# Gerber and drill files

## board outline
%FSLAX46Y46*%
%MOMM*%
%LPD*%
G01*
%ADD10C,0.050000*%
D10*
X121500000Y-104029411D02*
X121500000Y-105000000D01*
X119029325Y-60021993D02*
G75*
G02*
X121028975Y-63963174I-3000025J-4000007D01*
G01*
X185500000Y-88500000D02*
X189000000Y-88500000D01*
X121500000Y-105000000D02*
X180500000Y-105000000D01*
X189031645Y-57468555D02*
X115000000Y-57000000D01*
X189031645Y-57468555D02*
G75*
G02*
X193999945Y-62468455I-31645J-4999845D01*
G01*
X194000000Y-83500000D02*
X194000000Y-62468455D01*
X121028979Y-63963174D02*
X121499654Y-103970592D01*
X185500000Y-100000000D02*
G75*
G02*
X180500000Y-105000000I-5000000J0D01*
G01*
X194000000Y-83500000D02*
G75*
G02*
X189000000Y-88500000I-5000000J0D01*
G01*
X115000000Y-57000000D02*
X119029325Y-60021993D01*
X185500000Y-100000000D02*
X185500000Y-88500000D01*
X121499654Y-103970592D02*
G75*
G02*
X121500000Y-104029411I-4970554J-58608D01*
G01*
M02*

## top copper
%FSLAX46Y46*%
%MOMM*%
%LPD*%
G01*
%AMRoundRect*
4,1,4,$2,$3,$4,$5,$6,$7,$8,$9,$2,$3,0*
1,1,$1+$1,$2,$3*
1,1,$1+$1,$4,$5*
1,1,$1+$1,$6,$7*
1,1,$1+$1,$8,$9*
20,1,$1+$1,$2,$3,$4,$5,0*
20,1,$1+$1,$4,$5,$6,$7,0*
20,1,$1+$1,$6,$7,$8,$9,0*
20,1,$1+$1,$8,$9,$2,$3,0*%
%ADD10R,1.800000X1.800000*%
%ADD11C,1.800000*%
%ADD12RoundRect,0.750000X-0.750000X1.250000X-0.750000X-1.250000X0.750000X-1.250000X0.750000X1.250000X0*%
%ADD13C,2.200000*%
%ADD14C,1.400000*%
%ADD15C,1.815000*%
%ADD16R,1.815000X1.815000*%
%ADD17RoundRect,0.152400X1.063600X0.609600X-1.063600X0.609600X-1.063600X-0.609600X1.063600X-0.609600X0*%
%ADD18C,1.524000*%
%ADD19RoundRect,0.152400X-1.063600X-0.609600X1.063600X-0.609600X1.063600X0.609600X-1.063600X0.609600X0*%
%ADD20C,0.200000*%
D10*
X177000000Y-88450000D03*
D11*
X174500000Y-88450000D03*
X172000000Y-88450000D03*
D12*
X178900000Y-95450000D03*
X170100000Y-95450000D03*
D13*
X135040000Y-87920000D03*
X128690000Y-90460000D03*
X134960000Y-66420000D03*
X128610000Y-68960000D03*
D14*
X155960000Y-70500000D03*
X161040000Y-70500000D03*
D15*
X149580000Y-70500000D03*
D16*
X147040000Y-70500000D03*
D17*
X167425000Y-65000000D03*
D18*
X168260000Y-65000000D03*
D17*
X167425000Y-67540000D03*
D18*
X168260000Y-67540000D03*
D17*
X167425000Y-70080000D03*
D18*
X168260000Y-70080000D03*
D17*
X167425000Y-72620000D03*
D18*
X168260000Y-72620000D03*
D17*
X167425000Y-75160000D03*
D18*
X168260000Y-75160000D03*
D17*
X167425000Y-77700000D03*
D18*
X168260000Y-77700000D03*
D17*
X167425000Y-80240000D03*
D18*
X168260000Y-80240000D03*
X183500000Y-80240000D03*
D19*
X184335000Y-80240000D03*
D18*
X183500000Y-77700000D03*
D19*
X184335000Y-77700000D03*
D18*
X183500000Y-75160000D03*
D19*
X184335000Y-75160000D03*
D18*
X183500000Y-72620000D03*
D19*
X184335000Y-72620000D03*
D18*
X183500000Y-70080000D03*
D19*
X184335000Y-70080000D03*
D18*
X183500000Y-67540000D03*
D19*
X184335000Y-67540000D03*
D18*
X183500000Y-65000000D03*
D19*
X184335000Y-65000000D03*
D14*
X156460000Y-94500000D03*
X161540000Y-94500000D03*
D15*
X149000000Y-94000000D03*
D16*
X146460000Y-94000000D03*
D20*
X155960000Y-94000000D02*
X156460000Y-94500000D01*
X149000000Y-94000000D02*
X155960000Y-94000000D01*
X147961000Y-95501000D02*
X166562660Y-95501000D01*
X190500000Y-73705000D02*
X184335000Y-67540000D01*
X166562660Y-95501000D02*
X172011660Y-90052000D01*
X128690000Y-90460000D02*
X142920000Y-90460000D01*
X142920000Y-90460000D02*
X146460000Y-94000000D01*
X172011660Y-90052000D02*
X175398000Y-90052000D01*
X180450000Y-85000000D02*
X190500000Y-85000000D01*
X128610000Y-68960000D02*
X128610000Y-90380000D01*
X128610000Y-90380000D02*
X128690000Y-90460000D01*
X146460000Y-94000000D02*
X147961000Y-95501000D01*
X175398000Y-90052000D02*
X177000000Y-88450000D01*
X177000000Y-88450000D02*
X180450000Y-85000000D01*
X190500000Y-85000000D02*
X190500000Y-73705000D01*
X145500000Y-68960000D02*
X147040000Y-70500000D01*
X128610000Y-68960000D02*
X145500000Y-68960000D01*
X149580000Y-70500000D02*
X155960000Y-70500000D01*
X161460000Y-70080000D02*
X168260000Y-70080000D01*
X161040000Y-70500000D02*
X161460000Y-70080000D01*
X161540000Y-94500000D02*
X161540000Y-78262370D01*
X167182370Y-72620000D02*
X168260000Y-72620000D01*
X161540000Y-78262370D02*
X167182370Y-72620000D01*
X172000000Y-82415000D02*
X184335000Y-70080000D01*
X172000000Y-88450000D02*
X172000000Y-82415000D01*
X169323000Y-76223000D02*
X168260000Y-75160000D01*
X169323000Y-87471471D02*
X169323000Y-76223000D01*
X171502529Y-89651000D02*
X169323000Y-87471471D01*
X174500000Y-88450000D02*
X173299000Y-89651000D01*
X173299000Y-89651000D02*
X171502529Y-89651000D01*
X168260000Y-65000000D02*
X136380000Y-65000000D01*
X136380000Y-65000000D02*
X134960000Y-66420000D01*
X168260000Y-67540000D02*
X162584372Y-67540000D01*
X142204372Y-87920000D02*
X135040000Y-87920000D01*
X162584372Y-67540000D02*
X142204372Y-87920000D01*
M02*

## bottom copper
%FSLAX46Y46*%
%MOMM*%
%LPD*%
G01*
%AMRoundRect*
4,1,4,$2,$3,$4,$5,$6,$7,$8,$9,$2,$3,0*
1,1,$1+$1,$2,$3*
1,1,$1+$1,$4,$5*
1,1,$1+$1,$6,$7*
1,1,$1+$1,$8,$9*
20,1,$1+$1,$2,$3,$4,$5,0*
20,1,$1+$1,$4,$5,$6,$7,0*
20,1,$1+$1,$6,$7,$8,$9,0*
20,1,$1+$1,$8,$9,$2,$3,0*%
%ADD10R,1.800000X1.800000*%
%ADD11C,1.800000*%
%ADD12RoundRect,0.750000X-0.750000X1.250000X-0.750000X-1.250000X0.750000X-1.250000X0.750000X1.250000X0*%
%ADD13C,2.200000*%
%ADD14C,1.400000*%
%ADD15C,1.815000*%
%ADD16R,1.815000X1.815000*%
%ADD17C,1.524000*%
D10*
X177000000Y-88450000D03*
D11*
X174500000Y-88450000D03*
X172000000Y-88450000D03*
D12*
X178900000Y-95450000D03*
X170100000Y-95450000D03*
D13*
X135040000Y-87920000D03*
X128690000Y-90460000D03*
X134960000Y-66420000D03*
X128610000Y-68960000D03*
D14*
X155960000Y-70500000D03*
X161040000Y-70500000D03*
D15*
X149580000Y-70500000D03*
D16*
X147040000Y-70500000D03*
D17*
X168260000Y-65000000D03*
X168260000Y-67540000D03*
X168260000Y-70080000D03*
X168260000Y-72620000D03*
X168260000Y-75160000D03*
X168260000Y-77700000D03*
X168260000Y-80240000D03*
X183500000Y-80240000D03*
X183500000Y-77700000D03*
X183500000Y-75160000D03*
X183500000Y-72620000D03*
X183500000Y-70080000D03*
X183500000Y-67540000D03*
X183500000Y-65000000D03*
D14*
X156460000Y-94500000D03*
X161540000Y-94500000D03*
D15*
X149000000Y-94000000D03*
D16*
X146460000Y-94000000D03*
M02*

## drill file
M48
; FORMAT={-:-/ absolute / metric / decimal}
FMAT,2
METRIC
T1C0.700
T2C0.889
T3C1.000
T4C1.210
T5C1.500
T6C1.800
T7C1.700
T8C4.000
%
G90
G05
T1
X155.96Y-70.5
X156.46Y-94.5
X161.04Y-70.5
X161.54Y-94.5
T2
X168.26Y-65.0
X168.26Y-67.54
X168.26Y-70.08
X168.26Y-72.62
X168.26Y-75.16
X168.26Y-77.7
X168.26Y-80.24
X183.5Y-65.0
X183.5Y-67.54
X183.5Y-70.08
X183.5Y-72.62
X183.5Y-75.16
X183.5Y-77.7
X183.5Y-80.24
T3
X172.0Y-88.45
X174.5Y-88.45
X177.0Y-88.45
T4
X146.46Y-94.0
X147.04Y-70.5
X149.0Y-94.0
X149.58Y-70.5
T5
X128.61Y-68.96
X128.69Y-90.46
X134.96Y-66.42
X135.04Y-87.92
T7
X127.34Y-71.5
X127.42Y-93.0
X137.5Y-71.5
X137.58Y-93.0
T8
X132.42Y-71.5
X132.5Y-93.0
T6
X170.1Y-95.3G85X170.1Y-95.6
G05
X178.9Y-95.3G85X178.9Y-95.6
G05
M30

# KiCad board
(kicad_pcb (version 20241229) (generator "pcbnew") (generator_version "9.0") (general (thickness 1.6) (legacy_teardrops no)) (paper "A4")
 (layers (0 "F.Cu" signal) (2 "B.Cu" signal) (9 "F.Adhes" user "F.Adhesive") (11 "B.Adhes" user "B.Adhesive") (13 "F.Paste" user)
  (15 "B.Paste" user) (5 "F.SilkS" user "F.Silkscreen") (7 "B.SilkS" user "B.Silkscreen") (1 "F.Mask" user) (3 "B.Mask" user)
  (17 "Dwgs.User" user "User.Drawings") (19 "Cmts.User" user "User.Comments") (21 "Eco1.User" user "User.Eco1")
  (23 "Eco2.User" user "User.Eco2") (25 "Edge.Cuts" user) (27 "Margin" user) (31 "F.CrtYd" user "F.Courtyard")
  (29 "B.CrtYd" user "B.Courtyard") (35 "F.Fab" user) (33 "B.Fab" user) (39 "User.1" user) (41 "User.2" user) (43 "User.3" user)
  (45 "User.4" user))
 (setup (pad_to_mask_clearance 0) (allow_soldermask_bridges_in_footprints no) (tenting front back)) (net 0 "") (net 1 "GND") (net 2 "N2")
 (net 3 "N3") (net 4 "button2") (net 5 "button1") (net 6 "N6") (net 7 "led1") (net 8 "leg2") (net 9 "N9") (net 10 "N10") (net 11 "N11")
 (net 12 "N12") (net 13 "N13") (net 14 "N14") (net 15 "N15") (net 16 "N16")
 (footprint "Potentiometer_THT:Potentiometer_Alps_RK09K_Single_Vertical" (layer "F.Cu") (at 177 88.45 -90)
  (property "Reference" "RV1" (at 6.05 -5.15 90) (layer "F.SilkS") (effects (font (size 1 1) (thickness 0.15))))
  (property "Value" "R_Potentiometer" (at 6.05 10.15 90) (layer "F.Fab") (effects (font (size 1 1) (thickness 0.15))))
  (pad "1" thru_hole rect (at 0 0 270) (size 1.8 1.8) (drill 1) (layers "*.Cu" "*.Mask") (remove_unused_layers no) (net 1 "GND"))
  (pad "2" thru_hole circle (at 0 2.5 270) (size 1.8 1.8) (drill 1) (layers "*.Cu" "*.Mask") (remove_unused_layers no) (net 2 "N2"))
  (pad "3" thru_hole circle (at 0 5 270) (size 1.8 1.8) (drill 1) (layers "*.Cu" "*.Mask") (remove_unused_layers no) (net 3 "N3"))
  (pad "MP" thru_hole roundrect (at 7 -1.9 270) (size 4 3) (drill oval 2.1 1.8) (layers "*.Cu" "*.Mask") (remove_unused_layers no)
   (roundrect_rratio 0.25))
  (pad "MP" thru_hole roundrect (at 7 6.9 270) (size 4 3) (drill oval 2.1 1.8) (layers "*.Cu" "*.Mask") (remove_unused_layers no)
   (roundrect_rratio 0.25)))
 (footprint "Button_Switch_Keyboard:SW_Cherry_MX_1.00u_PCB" (layer "F.Cu") (at 135.04 87.92)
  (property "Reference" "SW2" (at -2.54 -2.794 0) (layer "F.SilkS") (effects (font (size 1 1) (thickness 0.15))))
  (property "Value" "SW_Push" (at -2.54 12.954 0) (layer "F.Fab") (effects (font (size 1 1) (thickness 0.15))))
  (pad "" np_thru_hole circle (at -7.62 5.08) (size 1.7 1.7) (drill 1.7) (layers "*.Cu" "*.Mask"))
  (pad "" np_thru_hole circle (at -2.54 5.08) (size 4 4) (drill 4) (layers "*.Cu" "*.Mask"))
  (pad "" np_thru_hole circle (at 2.54 5.08) (size 1.7 1.7) (drill 1.7) (layers "*.Cu" "*.Mask"))
  (pad "1" thru_hole circle (at 0 0) (size 2.2 2.2) (drill 1.5) (layers "*.Cu" "*.Mask") (remove_unused_layers no) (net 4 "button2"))
  (pad "2" thru_hole circle (at -6.35 2.54) (size 2.2 2.2) (drill 1.5) (layers "*.Cu" "*.Mask") (remove_unused_layers no) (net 1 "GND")))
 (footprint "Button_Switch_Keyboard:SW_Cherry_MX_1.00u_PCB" (layer "F.Cu") (at 134.96 66.42)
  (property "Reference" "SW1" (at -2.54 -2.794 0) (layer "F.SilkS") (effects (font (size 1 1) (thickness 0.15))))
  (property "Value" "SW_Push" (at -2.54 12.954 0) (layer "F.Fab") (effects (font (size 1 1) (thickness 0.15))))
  (pad "" np_thru_hole circle (at -7.62 5.08) (size 1.7 1.7) (drill 1.7) (layers "*.Cu" "*.Mask"))
  (pad "" np_thru_hole circle (at -2.54 5.08) (size 4 4) (drill 4) (layers "*.Cu" "*.Mask"))
  (pad "" np_thru_hole circle (at 2.54 5.08) (size 1.7 1.7) (drill 1.7) (layers "*.Cu" "*.Mask"))
  (pad "1" thru_hole circle (at 0 0) (size 2.2 2.2) (drill 1.5) (layers "*.Cu" "*.Mask") (remove_unused_layers no) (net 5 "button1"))
  (pad "2" thru_hole circle (at -6.35 2.54) (size 2.2 2.2) (drill 1.5) (layers "*.Cu" "*.Mask") (remove_unused_layers no) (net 1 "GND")))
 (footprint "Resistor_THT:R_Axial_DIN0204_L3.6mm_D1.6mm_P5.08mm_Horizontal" (layer "F.Cu") (at 155.96 70.5)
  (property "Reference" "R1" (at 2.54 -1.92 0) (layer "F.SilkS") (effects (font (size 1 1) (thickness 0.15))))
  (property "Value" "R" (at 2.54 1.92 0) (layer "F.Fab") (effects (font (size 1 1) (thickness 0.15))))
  (pad "1" thru_hole circle (at 0 0) (size 1.4 1.4) (drill 0.7) (layers "*.Cu" "*.Mask") (remove_unused_layers no) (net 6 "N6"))
  (pad "2" thru_hole circle (at 5.08 0) (size 1.4 1.4) (drill 0.7) (layers "*.Cu" "*.Mask") (remove_unused_layers no) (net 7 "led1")))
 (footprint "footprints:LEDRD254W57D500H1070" (layer "F.Cu") (at 148.31 70.5)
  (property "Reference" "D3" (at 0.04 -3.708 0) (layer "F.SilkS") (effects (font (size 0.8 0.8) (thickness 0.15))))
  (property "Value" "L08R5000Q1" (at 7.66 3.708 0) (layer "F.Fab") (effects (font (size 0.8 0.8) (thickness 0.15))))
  (pad "A" thru_hole circle (at 1.27 0) (size 1.815 1.815) (drill 1.21) (layers "*.Cu" "*.Mask") (remove_unused_layers no) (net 6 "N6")
   (solder_mask_margin 0.102))
  (pad "C" thru_hole rect (at -1.27 0) (size 1.815 1.815) (drill 1.21) (layers "*.Cu" "*.Mask") (remove_unused_layers no) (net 1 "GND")
   (solder_mask_margin 0.102)))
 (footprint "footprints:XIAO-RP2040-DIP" (layer "F.Cu") (at 175.88 72.62 90)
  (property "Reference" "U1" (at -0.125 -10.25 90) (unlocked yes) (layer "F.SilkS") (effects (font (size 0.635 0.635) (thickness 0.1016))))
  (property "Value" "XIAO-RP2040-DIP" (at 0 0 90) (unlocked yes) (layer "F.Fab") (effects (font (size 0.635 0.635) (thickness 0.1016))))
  (pad "1" smd roundrect (at 7.62 -8.455 180) (size 2.432 1.524) (layers "F.Cu" "F.Mask") (roundrect_rratio 0.1) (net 5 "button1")
   (thermal_bridge_angle 45))
  (pad "1" thru_hole circle (at 7.62 -7.62 180) (size 1.524 1.524) (drill 0.889) (layers "*.Cu" "*.Mask") (remove_unused_layers no)
   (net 5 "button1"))
  (pad "2" smd roundrect (at 5.08 -8.455 180) (size 2.432 1.524) (layers "F.Cu" "F.Mask") (roundrect_rratio 0.1) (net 4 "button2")
   (thermal_bridge_angle 45))
  (pad "2" thru_hole circle (at 5.08 -7.62 180) (size 1.524 1.524) (drill 0.889) (layers "*.Cu" "*.Mask") (remove_unused_layers no)
   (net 4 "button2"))
  (pad "3" smd roundrect (at 2.54 -8.455 180) (size 2.432 1.524) (layers "F.Cu" "F.Mask") (roundrect_rratio 0.1) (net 7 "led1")
   (thermal_bridge_angle 45))
  (pad "3" thru_hole circle (at 2.54 -7.62 180) (size 1.524 1.524) (drill 0.889) (layers "*.Cu" "*.Mask") (remove_unused_layers no)
   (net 7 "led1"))
  (pad "4" smd roundrect (at 0 -8.455 180) (size 2.432 1.524) (layers "F.Cu" "F.Mask") (roundrect_rratio 0.1) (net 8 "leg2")
   (thermal_bridge_angle 45))
  (pad "4" thru_hole circle (at 0 -7.62 180) (size 1.524 1.524) (drill 0.889) (layers "*.Cu" "*.Mask") (remove_unused_layers no)
   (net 8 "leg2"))
  (pad "5" smd roundrect (at -2.54 -8.455 180) (size 2.432 1.524) (layers "F.Cu" "F.Mask") (roundrect_rratio 0.1) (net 2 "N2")
   (thermal_bridge_angle 45))
  (pad "5" thru_hole circle (at -2.54 -7.62 180) (size 1.524 1.524) (drill 0.889) (layers "*.Cu" "*.Mask") (remove_unused_layers no)
   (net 2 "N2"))
  (pad "6" smd roundrect (at -5.08 -8.455 180) (size 2.432 1.524) (layers "F.Cu" "F.Mask") (roundrect_rratio 0.1) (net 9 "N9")
   (thermal_bridge_angle 45))
  (pad "6" thru_hole circle (at -5.08 -7.62 180) (size 1.524 1.524) (drill 0.889) (layers "*.Cu" "*.Mask") (remove_unused_layers no)
   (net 9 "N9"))
  (pad "7" smd roundrect (at -7.62 -8.455 180) (size 2.432 1.524) (layers "F.Cu" "F.Mask") (roundrect_rratio 0.1) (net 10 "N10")
   (thermal_bridge_angle 45))
  (pad "7" thru_hole circle (at -7.62 -7.62 180) (size 1.524 1.524) (drill 0.889) (layers "*.Cu" "*.Mask") (remove_unused_layers no)
   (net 10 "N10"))
  (pad "8" thru_hole circle (at -7.62 7.62) (size 1.524 1.524) (drill 0.889) (layers "*.Cu" "*.Mask") (remove_unused_layers no)
   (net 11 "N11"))
  (pad "8" smd roundrect (at -7.62 8.455) (size 2.432 1.524) (layers "F.Cu" "F.Mask") (roundrect_rratio 0.1) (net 11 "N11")
   (thermal_bridge_angle 45))
  (pad "9" thru_hole circle (at -5.08 7.62) (size 1.524 1.524) (drill 0.889) (layers "*.Cu" "*.Mask") (remove_unused_layers no)
   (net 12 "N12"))
  (pad "9" smd roundrect (at -5.08 8.455) (size 2.432 1.524) (layers "F.Cu" "F.Mask") (roundrect_rratio 0.1) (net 12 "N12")
   (thermal_bridge_angle 45))
  (pad "10" thru_hole circle (at -2.54 7.62) (size 1.524 1.524) (drill 0.889) (layers "*.Cu" "*.Mask") (remove_unused_layers no)
   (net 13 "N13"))
  (pad "10" smd roundrect (at -2.54 8.455) (size 2.432 1.524) (layers "F.Cu" "F.Mask") (roundrect_rratio 0.1) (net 13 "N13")
   (thermal_bridge_angle 45))
  (pad "11" thru_hole circle (at 0 7.62) (size 1.524 1.524) (drill 0.889) (layers "*.Cu" "*.Mask") (remove_unused_layers no) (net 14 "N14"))
  (pad "11" smd roundrect (at 0 8.455) (size 2.432 1.524) (layers "F.Cu" "F.Mask") (roundrect_rratio 0.1) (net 14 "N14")
   (thermal_bridge_angle 45))
  (pad "12" thru_hole circle (at 2.54 7.62) (size 1.524 1.524) (drill 0.889) (layers "*.Cu" "*.Mask") (remove_unused_layers no) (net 3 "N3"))
  (pad "12" smd roundrect (at 2.54 8.455) (size 2.432 1.524) (layers "F.Cu" "F.Mask") (roundrect_rratio 0.1) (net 3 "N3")
   (thermal_bridge_angle 45))
  (pad "13" thru_hole circle (at 5.08 7.62) (size 1.524 1.524) (drill 0.889) (layers "*.Cu" "*.Mask") (remove_unused_layers no)
   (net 1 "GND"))
  (pad "13" smd roundrect (at 5.08 8.455) (size 2.432 1.524) (layers "F.Cu" "F.Mask") (roundrect_rratio 0.1) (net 1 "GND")
   (thermal_bridge_angle 45))
  (pad "14" thru_hole circle (at 7.62 7.62) (size 1.524 1.524) (drill 0.889) (layers "*.Cu" "*.Mask") (remove_unused_layers no)
   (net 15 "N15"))
  (pad "14" smd roundrect (at 7.62 8.455) (size 2.432 1.524) (layers "F.Cu" "F.Mask") (roundrect_rratio 0.1) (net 15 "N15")
   (thermal_bridge_angle 45)))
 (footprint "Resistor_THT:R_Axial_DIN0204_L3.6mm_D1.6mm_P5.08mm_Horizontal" (layer "F.Cu") (at 156.46 94.5)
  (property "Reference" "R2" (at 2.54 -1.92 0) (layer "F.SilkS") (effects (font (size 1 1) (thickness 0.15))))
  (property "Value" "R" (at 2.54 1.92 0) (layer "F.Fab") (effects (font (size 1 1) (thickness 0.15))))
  (pad "1" thru_hole circle (at 0 0) (size 1.4 1.4) (drill 0.7) (layers "*.Cu" "*.Mask") (remove_unused_layers no) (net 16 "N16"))
  (pad "2" thru_hole circle (at 5.08 0) (size 1.4 1.4) (drill 0.7) (layers "*.Cu" "*.Mask") (remove_unused_layers no) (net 8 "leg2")))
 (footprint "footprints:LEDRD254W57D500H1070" (layer "F.Cu") (at 147.73 94)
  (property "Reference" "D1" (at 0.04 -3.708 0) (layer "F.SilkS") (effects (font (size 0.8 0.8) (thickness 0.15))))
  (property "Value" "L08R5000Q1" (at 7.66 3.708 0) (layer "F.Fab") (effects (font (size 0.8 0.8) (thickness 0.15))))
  (pad "A" thru_hole circle (at 1.27 0) (size 1.815 1.815) (drill 1.21) (layers "*.Cu" "*.Mask") (remove_unused_layers no) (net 16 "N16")
   (solder_mask_margin 0.102))
  (pad "C" thru_hole rect (at -1.27 0) (size 1.815 1.815) (drill 1.21) (layers "*.Cu" "*.Mask") (remove_unused_layers no) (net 1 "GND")
   (solder_mask_margin 0.102)))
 (gr_line (start 121.5 104.029411) (end 121.5 105) (stroke (width 0.05) (type default)) (layer "Edge.Cuts"))
 (gr_arc (start 119.029325 60.021993) (mid 120.488231 61.759659) (end 121.028979 63.963174) (stroke (width 0.05) (type default))
  (layer "Edge.Cuts"))
 (gr_line (start 185.5 88.5) (end 189 88.5) (stroke (width 0.05) (type default)) (layer "Edge.Cuts"))
 (gr_line (start 121.5 105) (end 180.5 105) (stroke (width 0.05) (type default)) (layer "Edge.Cuts"))
 (gr_line (start 189.031645 57.468555) (end 115 57) (stroke (width 0.05) (type default)) (layer "Edge.Cuts"))
 (gr_arc (start 189.031645 57.468555) (mid 192.546721 58.944124) (end 194 62.468455) (stroke (width 0.05) (type default))
  (layer "Edge.Cuts"))
 (gr_line (start 194 83.5) (end 194 62.468455) (stroke (width 0.05) (type default)) (layer "Edge.Cuts"))
 (gr_line (start 121.028979 63.963174) (end 121.499654 103.970592) (stroke (width 0.05) (type default)) (layer "Edge.Cuts"))
 (gr_arc (start 185.5 100) (mid 184.035534 103.535534) (end 180.5 105) (stroke (width 0.05) (type default)) (layer "Edge.Cuts"))
 (gr_arc (start 194 83.5) (mid 192.535534 87.035534) (end 189 88.5) (stroke (width 0.05) (type default)) (layer "Edge.Cuts"))
 (gr_line (start 115 57) (end 119.029325 60.021993) (stroke (width 0.05) (type default)) (layer "Edge.Cuts"))
 (gr_line (start 185.5 100) (end 185.5 88.5) (stroke (width 0.05) (type default)) (layer "Edge.Cuts"))
 (gr_arc (start 121.499654 103.970592) (mid 121.499914 104.000001) (end 121.5 104.029411) (stroke (width 0.05) (type default))
  (layer "Edge.Cuts"))
 (segment (start 155.96 94) (end 156.46 94.5) (width 0.2) (layer "F.Cu") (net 16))
 (segment (start 149 94) (end 155.96 94) (width 0.2) (layer "F.Cu") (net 16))
 (segment (start 147.961 95.501) (end 166.56266 95.501) (width 0.2) (layer "F.Cu") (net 1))
 (segment (start 190.5 73.705) (end 184.335 67.54) (width 0.2) (layer "F.Cu") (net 1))
 (segment (start 166.56266 95.501) (end 172.01166 90.052) (width 0.2) (layer "F.Cu") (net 1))
 (segment (start 128.69 90.46) (end 142.92 90.46) (width 0.2) (layer "F.Cu") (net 1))
 (segment (start 142.92 90.46) (end 146.46 94) (width 0.2) (layer "F.Cu") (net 1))
 (segment (start 172.01166 90.052) (end 175.398 90.052) (width 0.2) (layer "F.Cu") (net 1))
 (segment (start 180.45 85) (end 190.5 85) (width 0.2) (layer "F.Cu") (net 1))
 (segment (start 128.61 68.96) (end 128.61 90.38) (width 0.2) (layer "F.Cu") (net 1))
 (segment (start 128.61 90.38) (end 128.69 90.46) (width 0.2) (layer "F.Cu") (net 1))
 (segment (start 146.46 94) (end 147.961 95.501) (width 0.2) (layer "F.Cu") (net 1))
 (segment (start 175.398 90.052) (end 177 88.45) (width 0.2) (layer "F.Cu") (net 1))
 (segment (start 177 88.45) (end 180.45 85) (width 0.2) (layer "F.Cu") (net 1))
 (segment (start 190.5 85) (end 190.5 73.705) (width 0.2) (layer "F.Cu") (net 1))
 (segment (start 145.5 68.96) (end 147.04 70.5) (width 0.2) (layer "F.Cu") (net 1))
 (segment (start 128.61 68.96) (end 145.5 68.96) (width 0.2) (layer "F.Cu") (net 1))
 (segment (start 149.58 70.5) (end 155.96 70.5) (width 0.2) (layer "F.Cu") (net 6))
 (segment (start 161.46 70.08) (end 168.26 70.08) (width 0.2) (layer "F.Cu") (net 7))
 (segment (start 161.04 70.5) (end 161.46 70.08) (width 0.2) (layer "F.Cu") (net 7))
 (segment (start 161.54 94.5) (end 161.54 78.26237) (width 0.2) (layer "F.Cu") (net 8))
 (segment (start 167.18237 72.62) (end 168.26 72.62) (width 0.2) (layer "F.Cu") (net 8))
 (segment (start 161.54 78.26237) (end 167.18237 72.62) (width 0.2) (layer "F.Cu") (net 8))
 (segment (start 172 82.415) (end 184.335 70.08) (width 0.2) (layer "F.Cu") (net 3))
 (segment (start 172 88.45) (end 172 82.415) (width 0.2) (layer "F.Cu") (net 3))
 (segment (start 169.323 76.223) (end 168.26 75.16) (width 0.2) (layer "F.Cu") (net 2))
 (segment (start 169.323 87.471471) (end 169.323 76.223) (width 0.2) (layer "F.Cu") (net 2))
 (segment (start 171.502529 89.651) (end 169.323 87.471471) (width 0.2) (layer "F.Cu") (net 2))
 (segment (start 174.5 88.45) (end 173.299 89.651) (width 0.2) (layer "F.Cu") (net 2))
 (segment (start 173.299 89.651) (end 171.502529 89.651) (width 0.2) (layer "F.Cu") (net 2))
 (segment (start 168.26 65) (end 136.38 65) (width 0.2) (layer "F.Cu") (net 5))
 (segment (start 136.38 65) (end 134.96 66.42) (width 0.2) (layer "F.Cu") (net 5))
 (segment (start 168.26 67.54) (end 162.584372 67.54) (width 0.2) (layer "F.Cu") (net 4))
 (segment (start 142.204372 87.92) (end 135.04 87.92) (width 0.2) (layer "F.Cu") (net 4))
 (segment (start 162.584372 67.54) (end 142.204372 87.92) (width 0.2) (layer "F.Cu") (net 4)))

